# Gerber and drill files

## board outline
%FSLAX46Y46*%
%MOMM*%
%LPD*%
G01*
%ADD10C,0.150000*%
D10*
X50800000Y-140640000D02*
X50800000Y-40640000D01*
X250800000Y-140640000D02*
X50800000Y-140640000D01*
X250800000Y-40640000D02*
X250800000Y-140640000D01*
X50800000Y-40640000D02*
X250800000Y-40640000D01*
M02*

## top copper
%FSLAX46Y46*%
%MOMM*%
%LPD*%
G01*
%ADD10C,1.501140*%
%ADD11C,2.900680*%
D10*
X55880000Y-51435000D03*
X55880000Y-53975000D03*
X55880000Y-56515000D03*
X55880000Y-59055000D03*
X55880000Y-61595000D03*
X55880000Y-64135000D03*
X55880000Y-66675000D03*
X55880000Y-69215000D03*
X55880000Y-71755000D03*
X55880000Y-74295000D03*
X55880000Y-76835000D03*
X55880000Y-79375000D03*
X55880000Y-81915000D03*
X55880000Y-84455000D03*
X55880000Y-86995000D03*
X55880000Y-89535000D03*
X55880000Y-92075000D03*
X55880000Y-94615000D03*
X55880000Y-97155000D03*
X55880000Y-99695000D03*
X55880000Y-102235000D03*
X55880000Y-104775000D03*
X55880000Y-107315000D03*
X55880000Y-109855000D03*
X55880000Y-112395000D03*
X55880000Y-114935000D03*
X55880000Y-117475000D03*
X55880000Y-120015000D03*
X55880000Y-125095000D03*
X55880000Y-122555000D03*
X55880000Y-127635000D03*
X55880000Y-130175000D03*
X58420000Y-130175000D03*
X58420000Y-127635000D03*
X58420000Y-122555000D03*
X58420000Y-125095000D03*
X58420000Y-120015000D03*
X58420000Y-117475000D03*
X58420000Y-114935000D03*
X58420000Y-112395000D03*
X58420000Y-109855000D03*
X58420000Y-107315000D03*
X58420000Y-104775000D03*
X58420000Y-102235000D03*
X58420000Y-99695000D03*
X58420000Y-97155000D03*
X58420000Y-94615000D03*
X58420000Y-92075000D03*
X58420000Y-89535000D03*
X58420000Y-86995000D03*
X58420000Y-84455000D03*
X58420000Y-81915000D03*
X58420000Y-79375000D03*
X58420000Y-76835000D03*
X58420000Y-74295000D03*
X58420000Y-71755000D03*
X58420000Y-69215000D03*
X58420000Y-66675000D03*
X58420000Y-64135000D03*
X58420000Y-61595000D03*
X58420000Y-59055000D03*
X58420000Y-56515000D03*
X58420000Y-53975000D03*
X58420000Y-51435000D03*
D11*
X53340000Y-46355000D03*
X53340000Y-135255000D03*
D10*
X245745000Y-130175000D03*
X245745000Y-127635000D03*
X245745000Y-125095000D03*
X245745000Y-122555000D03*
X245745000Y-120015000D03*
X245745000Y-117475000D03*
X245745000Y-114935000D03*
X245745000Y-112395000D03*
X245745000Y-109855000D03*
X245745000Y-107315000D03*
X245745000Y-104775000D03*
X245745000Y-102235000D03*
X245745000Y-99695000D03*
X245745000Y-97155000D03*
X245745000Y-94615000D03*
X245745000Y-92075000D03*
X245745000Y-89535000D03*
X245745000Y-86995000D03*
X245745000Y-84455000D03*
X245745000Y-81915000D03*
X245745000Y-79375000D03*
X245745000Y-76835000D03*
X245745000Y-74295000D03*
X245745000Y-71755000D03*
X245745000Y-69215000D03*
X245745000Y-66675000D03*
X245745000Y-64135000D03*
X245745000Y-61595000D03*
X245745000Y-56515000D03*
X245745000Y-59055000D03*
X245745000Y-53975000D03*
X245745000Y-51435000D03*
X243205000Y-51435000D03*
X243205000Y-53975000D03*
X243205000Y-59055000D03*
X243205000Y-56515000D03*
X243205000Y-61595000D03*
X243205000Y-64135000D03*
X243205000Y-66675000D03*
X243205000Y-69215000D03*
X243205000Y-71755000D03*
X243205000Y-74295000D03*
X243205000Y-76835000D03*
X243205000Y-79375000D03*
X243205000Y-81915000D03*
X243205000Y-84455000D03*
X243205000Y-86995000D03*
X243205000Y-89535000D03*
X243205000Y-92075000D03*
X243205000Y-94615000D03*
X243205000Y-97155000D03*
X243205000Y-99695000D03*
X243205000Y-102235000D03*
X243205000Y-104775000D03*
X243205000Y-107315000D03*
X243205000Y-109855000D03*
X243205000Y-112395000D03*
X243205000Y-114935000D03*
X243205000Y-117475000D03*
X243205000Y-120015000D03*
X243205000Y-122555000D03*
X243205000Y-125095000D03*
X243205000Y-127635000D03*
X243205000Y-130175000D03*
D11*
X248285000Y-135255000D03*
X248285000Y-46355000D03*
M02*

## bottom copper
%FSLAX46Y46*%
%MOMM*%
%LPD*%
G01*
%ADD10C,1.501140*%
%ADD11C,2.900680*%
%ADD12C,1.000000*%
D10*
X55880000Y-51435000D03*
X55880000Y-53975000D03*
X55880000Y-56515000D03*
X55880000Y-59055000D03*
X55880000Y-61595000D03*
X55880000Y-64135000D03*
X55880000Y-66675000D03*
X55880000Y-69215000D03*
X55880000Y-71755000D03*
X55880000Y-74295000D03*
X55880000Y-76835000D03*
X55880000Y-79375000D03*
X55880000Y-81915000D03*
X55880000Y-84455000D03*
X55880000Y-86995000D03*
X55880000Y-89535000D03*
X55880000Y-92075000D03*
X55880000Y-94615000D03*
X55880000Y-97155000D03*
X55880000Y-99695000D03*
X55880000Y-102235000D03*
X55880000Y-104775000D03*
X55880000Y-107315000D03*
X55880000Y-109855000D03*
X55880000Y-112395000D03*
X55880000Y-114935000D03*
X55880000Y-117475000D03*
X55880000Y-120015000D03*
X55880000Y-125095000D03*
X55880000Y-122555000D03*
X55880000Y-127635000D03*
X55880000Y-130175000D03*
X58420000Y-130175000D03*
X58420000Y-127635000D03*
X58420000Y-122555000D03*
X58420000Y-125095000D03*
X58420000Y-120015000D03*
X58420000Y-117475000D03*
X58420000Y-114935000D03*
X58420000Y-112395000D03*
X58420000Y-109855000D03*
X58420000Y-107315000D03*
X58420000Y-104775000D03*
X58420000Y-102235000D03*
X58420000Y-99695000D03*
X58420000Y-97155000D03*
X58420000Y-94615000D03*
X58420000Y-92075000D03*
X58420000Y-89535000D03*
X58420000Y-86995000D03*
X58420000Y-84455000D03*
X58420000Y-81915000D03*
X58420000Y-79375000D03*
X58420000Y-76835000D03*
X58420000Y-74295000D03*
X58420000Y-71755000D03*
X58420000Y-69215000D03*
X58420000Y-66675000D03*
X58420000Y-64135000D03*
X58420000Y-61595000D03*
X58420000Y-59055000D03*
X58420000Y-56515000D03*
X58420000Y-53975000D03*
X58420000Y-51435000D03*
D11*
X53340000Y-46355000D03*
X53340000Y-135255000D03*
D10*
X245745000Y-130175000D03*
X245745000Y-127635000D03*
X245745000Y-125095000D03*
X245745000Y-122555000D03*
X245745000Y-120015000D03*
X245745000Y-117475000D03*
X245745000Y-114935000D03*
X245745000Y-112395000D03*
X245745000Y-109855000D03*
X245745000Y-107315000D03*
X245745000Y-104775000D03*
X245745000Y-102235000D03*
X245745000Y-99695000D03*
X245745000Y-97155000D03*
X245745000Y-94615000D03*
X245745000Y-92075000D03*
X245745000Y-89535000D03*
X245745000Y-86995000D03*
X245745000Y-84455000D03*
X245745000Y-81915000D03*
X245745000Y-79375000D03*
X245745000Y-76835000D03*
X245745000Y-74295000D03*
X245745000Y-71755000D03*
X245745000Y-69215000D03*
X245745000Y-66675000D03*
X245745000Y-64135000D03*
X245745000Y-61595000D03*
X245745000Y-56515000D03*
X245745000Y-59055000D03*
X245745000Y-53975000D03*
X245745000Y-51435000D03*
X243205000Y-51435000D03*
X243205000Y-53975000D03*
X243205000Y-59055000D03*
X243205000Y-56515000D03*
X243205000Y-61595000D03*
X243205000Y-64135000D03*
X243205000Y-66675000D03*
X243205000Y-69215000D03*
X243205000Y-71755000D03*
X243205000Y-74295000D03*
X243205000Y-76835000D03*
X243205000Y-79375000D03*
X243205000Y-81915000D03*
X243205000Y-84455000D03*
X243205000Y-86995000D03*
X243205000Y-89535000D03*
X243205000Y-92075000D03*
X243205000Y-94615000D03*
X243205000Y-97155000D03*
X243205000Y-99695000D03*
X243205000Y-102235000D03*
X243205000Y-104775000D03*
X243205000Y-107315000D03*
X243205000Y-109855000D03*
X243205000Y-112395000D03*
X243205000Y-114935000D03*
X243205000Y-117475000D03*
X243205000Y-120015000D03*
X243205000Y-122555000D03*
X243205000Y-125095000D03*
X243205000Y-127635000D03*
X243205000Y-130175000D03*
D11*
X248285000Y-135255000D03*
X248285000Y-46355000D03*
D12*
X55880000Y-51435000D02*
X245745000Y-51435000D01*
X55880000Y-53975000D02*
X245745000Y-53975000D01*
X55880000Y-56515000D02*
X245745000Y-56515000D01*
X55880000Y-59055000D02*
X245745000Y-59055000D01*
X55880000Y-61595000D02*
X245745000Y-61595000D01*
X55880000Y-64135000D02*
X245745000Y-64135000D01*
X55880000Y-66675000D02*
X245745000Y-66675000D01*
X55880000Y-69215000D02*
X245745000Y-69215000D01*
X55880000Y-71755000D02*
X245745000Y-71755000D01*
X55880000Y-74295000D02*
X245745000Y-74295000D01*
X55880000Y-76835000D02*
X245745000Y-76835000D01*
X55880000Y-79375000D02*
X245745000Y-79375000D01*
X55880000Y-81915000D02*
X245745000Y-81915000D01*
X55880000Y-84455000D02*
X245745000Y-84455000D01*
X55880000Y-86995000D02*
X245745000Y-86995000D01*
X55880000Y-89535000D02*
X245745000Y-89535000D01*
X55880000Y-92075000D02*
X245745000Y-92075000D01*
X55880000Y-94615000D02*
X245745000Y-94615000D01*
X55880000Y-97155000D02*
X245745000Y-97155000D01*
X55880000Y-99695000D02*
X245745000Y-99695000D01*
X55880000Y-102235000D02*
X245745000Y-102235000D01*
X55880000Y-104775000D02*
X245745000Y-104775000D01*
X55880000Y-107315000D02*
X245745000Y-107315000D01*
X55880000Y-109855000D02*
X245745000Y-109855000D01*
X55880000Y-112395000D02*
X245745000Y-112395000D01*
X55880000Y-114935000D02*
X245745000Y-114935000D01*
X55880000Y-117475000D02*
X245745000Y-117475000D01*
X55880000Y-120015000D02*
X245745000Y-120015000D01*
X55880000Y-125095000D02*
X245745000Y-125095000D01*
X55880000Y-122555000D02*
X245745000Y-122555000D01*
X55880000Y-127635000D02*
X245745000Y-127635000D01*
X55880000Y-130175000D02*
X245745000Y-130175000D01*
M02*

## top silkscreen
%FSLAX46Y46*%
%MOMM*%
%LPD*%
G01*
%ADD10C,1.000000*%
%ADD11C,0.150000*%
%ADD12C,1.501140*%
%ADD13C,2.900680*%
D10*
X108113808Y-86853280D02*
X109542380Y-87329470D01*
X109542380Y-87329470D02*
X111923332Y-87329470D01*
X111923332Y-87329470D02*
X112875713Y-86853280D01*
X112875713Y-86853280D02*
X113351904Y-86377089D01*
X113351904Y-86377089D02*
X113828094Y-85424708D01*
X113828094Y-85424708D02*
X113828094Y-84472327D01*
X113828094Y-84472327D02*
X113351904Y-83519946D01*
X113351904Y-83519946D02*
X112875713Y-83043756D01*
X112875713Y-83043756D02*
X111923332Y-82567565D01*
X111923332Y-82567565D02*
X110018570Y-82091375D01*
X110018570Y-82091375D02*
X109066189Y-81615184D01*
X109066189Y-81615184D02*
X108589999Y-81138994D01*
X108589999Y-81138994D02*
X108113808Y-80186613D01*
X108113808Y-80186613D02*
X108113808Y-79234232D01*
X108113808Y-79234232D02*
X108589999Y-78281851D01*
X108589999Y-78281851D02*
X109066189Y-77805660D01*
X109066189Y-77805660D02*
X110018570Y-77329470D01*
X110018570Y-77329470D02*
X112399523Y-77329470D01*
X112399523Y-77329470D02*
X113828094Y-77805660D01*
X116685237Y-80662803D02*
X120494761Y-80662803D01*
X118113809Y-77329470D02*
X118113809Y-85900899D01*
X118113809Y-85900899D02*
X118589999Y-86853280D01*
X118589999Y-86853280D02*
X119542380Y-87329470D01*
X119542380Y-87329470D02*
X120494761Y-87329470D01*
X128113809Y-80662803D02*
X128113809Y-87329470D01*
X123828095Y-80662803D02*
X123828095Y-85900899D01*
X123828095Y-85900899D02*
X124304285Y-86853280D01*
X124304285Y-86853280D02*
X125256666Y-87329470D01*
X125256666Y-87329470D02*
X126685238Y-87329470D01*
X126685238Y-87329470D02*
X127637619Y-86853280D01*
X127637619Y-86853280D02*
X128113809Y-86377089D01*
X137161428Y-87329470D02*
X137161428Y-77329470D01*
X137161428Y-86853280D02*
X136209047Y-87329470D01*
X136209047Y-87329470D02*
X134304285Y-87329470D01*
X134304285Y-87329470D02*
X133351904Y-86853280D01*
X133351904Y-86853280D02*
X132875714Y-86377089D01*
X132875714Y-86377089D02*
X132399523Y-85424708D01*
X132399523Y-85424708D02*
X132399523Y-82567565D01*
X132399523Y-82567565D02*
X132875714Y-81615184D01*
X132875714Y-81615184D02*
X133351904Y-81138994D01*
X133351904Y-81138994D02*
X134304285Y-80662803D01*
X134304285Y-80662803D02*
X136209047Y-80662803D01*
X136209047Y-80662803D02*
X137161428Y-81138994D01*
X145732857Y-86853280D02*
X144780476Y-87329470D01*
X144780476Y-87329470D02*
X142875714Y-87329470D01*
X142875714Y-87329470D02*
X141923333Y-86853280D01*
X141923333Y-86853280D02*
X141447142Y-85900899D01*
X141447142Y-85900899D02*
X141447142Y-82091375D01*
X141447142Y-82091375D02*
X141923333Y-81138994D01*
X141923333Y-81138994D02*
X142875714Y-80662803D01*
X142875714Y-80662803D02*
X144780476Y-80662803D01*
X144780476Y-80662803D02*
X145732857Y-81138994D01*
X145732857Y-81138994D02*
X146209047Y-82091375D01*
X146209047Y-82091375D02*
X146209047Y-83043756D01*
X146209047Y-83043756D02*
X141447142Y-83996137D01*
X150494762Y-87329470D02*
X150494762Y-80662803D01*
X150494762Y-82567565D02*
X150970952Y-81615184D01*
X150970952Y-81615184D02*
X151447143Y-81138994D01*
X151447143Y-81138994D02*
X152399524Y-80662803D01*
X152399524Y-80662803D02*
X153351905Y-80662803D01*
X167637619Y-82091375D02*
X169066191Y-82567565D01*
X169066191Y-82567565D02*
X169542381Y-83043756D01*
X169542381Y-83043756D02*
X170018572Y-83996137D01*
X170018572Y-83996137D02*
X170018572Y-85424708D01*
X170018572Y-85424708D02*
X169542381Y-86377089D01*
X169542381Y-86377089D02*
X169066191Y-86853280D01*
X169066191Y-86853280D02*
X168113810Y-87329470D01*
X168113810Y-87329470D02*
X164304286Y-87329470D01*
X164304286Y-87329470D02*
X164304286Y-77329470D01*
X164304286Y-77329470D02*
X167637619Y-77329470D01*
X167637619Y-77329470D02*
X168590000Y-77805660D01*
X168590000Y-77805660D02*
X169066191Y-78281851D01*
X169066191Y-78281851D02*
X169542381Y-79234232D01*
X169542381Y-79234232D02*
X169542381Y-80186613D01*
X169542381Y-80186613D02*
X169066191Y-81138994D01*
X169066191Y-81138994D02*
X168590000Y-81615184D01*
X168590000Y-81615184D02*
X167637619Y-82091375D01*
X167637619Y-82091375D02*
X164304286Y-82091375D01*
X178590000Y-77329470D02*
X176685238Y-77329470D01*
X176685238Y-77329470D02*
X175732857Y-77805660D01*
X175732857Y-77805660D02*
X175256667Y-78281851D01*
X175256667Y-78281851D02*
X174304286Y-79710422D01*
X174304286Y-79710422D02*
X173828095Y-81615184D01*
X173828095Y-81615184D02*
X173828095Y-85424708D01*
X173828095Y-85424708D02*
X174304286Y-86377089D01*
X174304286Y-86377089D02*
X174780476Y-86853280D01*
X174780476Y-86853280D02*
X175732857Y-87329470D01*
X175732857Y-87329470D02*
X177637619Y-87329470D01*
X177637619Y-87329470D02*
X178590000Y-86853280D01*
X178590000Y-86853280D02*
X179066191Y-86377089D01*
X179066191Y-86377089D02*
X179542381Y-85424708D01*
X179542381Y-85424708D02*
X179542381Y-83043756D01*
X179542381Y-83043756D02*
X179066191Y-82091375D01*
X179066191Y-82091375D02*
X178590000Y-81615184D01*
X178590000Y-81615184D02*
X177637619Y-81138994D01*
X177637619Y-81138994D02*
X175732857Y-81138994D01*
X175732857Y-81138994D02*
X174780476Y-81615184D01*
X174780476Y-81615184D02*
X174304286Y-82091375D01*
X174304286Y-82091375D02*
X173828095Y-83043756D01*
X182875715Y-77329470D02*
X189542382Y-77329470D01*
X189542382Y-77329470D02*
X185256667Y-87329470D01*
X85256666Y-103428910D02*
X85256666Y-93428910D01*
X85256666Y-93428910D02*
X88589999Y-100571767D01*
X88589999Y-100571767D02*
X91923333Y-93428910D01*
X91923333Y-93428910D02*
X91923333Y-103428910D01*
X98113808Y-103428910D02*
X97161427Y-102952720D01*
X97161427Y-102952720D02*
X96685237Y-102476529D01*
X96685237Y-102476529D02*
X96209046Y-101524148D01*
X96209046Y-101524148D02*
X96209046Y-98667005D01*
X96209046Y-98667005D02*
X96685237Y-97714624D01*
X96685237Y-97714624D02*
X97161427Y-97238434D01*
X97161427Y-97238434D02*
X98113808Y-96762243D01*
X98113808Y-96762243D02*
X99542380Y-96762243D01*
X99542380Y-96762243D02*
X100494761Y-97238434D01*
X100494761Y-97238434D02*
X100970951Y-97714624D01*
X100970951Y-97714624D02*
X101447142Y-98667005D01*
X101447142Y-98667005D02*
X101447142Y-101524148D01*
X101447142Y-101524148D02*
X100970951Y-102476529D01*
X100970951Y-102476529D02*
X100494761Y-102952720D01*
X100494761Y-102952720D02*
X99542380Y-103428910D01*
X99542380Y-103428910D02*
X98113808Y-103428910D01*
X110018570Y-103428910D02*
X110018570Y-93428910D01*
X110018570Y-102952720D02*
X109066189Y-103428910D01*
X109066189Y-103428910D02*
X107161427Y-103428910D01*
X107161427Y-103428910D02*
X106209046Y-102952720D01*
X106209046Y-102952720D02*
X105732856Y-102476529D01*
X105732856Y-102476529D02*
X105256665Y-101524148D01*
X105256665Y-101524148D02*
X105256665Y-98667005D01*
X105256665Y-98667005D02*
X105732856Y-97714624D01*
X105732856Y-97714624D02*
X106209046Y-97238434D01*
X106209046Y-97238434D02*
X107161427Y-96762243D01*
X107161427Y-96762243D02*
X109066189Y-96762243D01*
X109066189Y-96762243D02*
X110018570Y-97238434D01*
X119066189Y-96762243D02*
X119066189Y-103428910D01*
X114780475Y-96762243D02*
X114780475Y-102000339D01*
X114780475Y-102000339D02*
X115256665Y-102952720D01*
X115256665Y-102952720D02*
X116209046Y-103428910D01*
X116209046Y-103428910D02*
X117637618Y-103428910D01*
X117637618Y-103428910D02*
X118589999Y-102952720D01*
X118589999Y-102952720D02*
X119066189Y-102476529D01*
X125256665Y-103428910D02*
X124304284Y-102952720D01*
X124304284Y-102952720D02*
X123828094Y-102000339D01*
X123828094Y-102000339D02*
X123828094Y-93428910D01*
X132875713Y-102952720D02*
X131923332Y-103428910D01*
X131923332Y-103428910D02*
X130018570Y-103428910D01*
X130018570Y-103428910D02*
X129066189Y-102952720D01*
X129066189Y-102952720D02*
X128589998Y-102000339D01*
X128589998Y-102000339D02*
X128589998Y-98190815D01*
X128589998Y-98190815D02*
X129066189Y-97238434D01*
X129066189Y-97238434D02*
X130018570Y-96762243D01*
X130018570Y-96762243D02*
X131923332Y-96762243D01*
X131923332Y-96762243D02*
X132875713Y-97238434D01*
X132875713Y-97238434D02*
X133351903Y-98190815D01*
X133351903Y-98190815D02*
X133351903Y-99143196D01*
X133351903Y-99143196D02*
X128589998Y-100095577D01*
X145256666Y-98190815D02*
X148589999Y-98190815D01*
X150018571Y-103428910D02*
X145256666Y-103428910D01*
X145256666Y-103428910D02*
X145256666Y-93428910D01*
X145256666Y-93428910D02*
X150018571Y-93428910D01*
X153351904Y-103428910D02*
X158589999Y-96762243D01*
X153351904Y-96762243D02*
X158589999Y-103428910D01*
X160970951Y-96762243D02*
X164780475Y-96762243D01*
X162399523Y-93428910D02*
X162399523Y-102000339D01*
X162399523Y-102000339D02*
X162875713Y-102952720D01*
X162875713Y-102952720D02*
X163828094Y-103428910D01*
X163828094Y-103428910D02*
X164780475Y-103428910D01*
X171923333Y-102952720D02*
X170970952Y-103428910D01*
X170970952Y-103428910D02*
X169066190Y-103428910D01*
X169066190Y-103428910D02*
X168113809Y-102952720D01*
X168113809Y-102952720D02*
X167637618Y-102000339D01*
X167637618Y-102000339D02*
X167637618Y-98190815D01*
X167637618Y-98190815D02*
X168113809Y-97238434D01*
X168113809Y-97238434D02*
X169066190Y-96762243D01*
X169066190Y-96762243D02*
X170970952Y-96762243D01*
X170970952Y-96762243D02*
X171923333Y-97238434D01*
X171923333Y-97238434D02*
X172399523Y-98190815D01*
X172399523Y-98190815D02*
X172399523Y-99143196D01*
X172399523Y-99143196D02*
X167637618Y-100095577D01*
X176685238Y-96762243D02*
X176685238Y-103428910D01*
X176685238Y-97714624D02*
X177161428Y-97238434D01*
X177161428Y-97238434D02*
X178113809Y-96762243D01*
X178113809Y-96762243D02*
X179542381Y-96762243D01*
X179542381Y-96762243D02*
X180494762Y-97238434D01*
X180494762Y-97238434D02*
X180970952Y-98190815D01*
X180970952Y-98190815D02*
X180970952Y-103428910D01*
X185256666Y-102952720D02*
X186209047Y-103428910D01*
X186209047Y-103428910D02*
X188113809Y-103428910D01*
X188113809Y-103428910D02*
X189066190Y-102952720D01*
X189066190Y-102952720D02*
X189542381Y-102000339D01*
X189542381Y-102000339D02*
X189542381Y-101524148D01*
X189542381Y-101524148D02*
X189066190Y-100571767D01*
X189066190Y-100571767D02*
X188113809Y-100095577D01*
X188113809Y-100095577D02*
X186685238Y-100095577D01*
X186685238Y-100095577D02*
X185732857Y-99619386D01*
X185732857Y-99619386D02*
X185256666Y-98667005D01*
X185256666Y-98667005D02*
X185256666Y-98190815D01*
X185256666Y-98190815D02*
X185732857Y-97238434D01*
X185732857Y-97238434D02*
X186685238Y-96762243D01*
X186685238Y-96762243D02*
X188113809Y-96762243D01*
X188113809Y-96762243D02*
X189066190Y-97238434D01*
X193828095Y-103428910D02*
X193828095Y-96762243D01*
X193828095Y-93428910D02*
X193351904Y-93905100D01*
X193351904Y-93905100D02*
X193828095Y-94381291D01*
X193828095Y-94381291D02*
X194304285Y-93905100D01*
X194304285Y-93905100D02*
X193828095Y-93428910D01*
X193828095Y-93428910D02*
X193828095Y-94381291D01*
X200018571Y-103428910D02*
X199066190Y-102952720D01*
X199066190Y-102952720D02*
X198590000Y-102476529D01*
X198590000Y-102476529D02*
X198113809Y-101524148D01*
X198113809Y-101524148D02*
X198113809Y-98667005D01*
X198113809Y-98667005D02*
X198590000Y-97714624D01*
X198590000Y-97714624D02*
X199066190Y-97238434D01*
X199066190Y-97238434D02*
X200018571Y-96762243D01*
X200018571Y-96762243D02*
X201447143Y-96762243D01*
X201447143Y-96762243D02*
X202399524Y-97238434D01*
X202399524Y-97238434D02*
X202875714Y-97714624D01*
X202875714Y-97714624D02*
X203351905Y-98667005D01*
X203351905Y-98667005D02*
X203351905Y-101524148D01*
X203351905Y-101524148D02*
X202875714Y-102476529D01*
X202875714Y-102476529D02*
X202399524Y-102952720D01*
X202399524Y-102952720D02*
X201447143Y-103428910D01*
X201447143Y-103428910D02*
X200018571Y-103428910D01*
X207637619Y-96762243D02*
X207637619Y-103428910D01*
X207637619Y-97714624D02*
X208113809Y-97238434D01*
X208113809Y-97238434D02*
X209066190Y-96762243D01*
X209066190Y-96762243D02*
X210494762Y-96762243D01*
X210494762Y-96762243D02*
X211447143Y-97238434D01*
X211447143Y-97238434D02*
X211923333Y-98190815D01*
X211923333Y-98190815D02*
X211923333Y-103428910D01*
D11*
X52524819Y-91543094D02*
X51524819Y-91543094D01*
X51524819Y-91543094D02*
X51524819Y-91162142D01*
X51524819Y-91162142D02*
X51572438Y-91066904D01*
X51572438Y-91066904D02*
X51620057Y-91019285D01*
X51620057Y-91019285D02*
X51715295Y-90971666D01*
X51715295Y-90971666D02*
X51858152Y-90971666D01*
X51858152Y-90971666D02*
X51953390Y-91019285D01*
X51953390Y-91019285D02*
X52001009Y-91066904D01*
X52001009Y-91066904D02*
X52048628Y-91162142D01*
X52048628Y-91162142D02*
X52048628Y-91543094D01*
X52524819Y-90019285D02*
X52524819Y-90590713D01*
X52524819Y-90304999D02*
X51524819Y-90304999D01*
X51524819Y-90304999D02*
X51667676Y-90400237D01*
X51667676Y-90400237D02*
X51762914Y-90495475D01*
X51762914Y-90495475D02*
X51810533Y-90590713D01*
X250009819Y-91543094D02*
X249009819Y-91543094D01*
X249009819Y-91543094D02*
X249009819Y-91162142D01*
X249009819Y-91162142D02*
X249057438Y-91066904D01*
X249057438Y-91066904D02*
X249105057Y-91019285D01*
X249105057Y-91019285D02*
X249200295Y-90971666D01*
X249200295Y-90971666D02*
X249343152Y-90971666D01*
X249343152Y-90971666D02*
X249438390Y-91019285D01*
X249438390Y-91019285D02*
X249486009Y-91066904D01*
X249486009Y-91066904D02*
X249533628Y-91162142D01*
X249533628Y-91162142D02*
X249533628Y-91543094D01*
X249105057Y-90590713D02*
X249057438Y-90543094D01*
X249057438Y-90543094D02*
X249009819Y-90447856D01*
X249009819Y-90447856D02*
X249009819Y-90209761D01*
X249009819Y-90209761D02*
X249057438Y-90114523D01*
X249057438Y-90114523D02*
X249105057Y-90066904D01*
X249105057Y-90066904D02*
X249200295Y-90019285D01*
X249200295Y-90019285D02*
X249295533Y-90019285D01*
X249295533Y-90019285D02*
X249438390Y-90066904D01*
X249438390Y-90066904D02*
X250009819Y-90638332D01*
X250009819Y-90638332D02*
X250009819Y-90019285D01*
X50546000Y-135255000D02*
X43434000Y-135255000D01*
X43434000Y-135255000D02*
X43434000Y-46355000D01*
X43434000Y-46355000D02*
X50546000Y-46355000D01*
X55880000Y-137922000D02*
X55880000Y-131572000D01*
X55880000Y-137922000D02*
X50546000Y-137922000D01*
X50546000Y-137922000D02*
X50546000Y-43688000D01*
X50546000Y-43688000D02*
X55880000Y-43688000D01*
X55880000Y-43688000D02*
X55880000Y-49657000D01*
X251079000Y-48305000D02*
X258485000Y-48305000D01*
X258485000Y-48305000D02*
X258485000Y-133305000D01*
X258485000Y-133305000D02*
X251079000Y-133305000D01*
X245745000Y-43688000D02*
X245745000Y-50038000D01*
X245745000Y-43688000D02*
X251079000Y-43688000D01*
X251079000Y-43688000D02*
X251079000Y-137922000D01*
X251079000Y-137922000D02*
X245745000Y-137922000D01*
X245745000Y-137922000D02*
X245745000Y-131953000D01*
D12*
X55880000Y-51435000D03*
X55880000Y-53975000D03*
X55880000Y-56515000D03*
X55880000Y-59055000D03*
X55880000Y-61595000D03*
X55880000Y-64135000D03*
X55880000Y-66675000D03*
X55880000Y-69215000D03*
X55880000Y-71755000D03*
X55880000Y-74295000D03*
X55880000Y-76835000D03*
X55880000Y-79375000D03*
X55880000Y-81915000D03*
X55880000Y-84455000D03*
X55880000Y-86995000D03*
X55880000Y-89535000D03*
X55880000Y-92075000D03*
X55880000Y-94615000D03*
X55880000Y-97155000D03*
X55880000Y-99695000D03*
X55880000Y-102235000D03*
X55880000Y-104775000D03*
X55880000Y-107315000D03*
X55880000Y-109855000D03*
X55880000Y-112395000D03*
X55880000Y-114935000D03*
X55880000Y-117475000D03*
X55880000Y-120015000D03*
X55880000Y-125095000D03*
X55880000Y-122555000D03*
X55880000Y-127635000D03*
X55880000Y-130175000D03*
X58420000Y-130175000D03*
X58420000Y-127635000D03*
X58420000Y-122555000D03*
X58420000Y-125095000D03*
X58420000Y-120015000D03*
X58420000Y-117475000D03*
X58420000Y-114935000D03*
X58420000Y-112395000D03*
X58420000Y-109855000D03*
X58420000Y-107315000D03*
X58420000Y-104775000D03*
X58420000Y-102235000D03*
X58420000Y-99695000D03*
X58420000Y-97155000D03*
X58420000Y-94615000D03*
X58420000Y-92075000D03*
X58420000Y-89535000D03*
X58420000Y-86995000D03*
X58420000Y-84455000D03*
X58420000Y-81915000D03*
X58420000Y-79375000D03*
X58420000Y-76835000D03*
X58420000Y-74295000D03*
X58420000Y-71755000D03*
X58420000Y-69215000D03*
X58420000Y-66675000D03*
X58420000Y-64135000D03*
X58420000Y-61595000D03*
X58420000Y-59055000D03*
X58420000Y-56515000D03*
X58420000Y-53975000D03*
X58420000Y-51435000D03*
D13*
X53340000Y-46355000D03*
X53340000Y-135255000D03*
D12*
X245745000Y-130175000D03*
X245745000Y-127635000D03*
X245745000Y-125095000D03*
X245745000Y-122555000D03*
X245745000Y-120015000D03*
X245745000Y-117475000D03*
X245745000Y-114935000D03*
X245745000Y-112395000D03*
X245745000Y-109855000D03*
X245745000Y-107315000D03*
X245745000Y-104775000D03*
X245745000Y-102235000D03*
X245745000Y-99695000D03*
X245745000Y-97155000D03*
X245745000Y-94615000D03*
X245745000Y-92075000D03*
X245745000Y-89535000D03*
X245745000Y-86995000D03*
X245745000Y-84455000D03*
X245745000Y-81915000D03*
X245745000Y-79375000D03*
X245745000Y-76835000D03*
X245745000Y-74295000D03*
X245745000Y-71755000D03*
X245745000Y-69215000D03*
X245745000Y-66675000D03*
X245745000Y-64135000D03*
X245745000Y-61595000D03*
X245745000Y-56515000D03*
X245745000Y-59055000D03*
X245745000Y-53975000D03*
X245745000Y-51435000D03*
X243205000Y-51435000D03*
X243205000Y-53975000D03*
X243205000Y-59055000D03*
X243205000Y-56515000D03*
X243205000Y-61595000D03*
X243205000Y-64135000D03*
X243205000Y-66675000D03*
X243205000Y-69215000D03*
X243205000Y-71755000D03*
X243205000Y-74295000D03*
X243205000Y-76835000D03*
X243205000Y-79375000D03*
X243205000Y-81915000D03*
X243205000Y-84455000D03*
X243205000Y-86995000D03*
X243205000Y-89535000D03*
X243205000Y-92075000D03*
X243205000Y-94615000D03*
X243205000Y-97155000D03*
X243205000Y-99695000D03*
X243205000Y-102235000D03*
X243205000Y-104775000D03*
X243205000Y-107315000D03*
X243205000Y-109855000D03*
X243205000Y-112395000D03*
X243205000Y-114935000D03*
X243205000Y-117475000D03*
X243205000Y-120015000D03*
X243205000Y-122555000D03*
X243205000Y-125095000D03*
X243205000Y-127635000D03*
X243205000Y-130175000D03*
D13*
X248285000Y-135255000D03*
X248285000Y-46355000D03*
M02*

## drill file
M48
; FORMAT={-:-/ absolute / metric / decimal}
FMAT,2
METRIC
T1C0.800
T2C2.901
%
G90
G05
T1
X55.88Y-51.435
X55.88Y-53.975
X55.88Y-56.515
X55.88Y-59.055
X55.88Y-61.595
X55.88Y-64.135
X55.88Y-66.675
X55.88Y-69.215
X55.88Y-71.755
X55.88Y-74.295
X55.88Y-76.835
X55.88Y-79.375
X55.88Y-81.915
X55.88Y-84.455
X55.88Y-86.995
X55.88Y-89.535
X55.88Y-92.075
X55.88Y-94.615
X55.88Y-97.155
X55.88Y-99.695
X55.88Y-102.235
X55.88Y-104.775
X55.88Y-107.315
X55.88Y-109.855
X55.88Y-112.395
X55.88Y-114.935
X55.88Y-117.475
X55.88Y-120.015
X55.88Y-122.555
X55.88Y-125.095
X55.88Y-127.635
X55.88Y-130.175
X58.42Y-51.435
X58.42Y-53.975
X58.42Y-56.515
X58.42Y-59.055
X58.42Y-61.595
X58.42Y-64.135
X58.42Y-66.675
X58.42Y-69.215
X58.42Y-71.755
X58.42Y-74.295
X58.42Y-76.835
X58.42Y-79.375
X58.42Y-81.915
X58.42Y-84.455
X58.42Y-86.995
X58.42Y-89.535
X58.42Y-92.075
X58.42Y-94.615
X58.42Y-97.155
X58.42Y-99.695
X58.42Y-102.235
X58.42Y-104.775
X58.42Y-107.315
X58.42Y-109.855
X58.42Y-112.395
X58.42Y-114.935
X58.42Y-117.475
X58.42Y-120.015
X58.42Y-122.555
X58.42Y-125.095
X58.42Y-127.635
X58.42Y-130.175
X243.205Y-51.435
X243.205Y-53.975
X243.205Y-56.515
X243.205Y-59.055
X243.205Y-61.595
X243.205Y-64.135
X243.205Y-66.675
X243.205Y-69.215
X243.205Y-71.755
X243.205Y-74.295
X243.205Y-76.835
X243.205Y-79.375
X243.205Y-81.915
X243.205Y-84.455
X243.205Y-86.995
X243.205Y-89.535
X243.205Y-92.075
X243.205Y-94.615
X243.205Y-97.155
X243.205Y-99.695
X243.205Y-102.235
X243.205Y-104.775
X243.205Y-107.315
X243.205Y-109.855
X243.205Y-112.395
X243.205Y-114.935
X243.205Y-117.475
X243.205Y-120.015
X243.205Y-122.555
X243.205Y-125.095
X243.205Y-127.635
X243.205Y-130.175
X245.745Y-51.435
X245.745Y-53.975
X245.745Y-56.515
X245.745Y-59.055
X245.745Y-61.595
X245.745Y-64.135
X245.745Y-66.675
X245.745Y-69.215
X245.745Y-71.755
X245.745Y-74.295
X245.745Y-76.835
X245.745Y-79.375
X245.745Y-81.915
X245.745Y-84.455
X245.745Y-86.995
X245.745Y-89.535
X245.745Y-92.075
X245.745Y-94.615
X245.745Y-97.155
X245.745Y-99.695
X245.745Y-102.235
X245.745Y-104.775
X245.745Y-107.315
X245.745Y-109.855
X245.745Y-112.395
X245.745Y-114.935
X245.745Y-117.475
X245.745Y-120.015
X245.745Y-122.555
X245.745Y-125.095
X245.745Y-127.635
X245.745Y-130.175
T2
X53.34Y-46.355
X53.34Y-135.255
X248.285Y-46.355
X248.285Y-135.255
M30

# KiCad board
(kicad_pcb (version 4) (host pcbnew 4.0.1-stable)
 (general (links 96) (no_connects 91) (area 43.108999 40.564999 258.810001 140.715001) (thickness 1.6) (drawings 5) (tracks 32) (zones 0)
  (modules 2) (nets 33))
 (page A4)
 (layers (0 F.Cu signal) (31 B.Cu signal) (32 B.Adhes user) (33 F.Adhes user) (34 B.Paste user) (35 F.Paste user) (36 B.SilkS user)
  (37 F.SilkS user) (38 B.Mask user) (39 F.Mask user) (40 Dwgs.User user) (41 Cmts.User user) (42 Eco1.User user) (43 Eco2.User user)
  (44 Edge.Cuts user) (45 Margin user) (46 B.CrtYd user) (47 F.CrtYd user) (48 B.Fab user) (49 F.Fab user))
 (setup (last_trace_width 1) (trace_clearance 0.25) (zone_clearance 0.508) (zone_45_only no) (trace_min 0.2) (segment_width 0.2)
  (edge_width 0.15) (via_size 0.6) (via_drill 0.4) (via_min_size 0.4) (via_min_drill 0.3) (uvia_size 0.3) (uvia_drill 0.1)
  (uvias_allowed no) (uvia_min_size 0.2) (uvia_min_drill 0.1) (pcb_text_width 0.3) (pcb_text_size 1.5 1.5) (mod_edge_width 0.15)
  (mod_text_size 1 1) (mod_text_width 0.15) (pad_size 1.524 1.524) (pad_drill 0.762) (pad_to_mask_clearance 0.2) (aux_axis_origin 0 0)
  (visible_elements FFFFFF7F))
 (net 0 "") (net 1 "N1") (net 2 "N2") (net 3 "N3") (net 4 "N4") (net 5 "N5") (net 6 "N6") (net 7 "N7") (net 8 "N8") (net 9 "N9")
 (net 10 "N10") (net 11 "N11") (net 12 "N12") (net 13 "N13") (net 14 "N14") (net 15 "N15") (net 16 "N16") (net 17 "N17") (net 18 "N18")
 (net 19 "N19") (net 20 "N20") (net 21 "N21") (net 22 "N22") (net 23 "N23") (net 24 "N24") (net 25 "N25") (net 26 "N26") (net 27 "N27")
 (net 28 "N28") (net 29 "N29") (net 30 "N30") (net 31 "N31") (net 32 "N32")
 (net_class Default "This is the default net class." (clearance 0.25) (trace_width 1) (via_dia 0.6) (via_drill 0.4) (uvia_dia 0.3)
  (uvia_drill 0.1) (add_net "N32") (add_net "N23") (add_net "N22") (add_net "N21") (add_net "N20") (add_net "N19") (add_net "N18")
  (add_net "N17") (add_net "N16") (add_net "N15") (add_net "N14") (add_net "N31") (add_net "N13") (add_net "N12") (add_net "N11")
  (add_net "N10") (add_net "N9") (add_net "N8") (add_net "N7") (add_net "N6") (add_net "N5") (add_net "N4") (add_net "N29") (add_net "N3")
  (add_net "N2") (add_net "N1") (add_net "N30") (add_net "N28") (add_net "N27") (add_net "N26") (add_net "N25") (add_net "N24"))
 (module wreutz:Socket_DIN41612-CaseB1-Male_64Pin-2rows (layer F.Cu) (at 57.15 90.805 270)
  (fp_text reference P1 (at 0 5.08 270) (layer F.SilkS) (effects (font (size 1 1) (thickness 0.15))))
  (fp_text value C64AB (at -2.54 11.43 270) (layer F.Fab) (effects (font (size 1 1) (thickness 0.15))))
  (fp_line (start 44.45 6.604) (end 44.45 13.716) (layer F.SilkS) (width 0.15))
  (fp_line (start 44.45 13.716) (end -44.45 13.716) (layer F.SilkS) (width 0.15))
  (fp_line (start -44.45 13.716) (end -44.45 6.604) (layer F.SilkS) (width 0.15))
  (fp_line (start 47.117 1.27) (end 40.767 1.27) (layer F.SilkS) (width 0.15))
  (fp_line (start 47.117 1.27) (end 47.117 6.604) (layer F.SilkS) (width 0.15))
  (fp_line (start 47.117 6.604) (end -47.117 6.604) (layer F.SilkS) (width 0.15))
  (fp_line (start -47.117 6.604) (end -47.117 1.27) (layer F.SilkS) (width 0.15))
  (fp_line (start -47.117 1.27) (end -41.148 1.27) (layer F.SilkS) (width 0.15))
  (pad B32 thru_hole circle (at -39.37 1.27 90) (size 1.50114 1.50114) (drill 0.8001) (layers *.Cu *.Mask F.SilkS) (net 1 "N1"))
  (pad B31 thru_hole circle (at -36.83 1.27 90) (size 1.50114 1.50114) (drill 0.8001) (layers *.Cu *.Mask F.SilkS) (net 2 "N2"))
  (pad B30 thru_hole circle (at -34.29 1.27 90) (size 1.50114 1.50114) (drill 0.8001) (layers *.Cu *.Mask F.SilkS) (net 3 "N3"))
  (pad B29 thru_hole circle (at -31.75 1.27 90) (size 1.50114 1.50114) (drill 0.8001) (layers *.Cu *.Mask F.SilkS) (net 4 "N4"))
  (pad B28 thru_hole circle (at -29.21 1.27 90) (size 1.50114 1.50114) (drill 0.8001) (layers *.Cu *.Mask F.SilkS) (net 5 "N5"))
  (pad B27 thru_hole circle (at -26.67 1.27 90) (size 1.50114 1.50114) (drill 0.8001) (layers *.Cu *.Mask F.SilkS) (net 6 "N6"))
  (pad B26 thru_hole circle (at -24.13 1.27 90) (size 1.50114 1.50114) (drill 0.8001) (layers *.Cu *.Mask F.SilkS) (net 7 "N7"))
  (pad B25 thru_hole circle (at -21.59 1.27 90) (size 1.50114 1.50114) (drill 0.8001) (layers *.Cu *.Mask F.SilkS) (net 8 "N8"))
  (pad B24 thru_hole circle (at -19.05 1.27 90) (size 1.50114 1.50114) (drill 0.8001) (layers *.Cu *.Mask F.SilkS) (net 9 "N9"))
  (pad B23 thru_hole circle (at -16.51 1.27 90) (size 1.50114 1.50114) (drill 0.8001) (layers *.Cu *.Mask F.SilkS) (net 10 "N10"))
  (pad B22 thru_hole circle (at -13.97 1.27 90) (size 1.50114 1.50114) (drill 0.8001) (layers *.Cu *.Mask F.SilkS) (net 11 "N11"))
  (pad B21 thru_hole circle (at -11.43 1.27 90) (size 1.50114 1.50114) (drill 0.8001) (layers *.Cu *.Mask F.SilkS) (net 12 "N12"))
  (pad B20 thru_hole circle (at -8.89 1.27 90) (size 1.50114 1.50114) (drill 0.8001) (layers *.Cu *.Mask F.SilkS) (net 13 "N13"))
  (pad B19 thru_hole circle (at -6.35 1.27 90) (size 1.50114 1.50114) (drill 0.8001) (layers *.Cu *.Mask F.SilkS) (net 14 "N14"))
  (pad B18 thru_hole circle (at -3.81 1.27 90) (size 1.50114 1.50114) (drill 0.8001) (layers *.Cu *.Mask F.SilkS) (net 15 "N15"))
  (pad B17 thru_hole circle (at -1.27 1.27 90) (size 1.50114 1.50114) (drill 0.8001) (layers *.Cu *.Mask F.SilkS) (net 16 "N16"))
  (pad B16 thru_hole circle (at 1.27 1.27 90) (size 1.50114 1.50114) (drill 0.8001) (layers *.Cu *.Mask F.SilkS) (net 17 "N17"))
  (pad B15 thru_hole circle (at 3.81 1.27 90) (size 1.50114 1.50114) (drill 0.8001) (layers *.Cu *.Mask F.SilkS) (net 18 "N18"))
  (pad B14 thru_hole circle (at 6.35 1.27 90) (size 1.50114 1.50114) (drill 0.8001) (layers *.Cu *.Mask F.SilkS) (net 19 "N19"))
  (pad B13 thru_hole circle (at 8.89 1.27 90) (size 1.50114 1.50114) (drill 0.8001) (layers *.Cu *.Mask F.SilkS) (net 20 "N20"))
  (pad B12 thru_hole circle (at 11.43 1.27 90) (size 1.50114 1.50114) (drill 0.8001) (layers *.Cu *.Mask F.SilkS) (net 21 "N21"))
  (pad B11 thru_hole circle (at 13.97 1.27 90) (size 1.50114 1.50114) (drill 0.8001) (layers *.Cu *.Mask F.SilkS) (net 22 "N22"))
  (pad B10 thru_hole circle (at 16.51 1.27 90) (size 1.50114 1.50114) (drill 0.8001) (layers *.Cu *.Mask F.SilkS) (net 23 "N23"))
  (pad B9 thru_hole circle (at 19.05 1.27 90) (size 1.50114 1.50114) (drill 0.8001) (layers *.Cu *.Mask F.SilkS) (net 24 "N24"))
  (pad B8 thru_hole circle (at 21.59 1.27 90) (size 1.50114 1.50114) (drill 0.8001) (layers *.Cu *.Mask F.SilkS) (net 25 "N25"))
  (pad B7 thru_hole circle (at 24.13 1.27 90) (size 1.50114 1.50114) (drill 0.8001) (layers *.Cu *.Mask F.SilkS) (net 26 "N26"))
  (pad B6 thru_hole circle (at 26.67 1.27 90) (size 1.50114 1.50114) (drill 0.8001) (layers *.Cu *.Mask F.SilkS) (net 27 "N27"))
  (pad B5 thru_hole circle (at 29.21 1.27 90) (size 1.50114 1.50114) (drill 0.8001) (layers *.Cu *.Mask F.SilkS) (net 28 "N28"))
  (pad B3 thru_hole circle (at 34.29 1.27 90) (size 1.50114 1.50114) (drill 0.8001) (layers *.Cu *.Mask F.SilkS) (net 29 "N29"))
  (pad B4 thru_hole circle (at 31.75 1.27 90) (size 1.50114 1.50114) (drill 0.8001) (layers *.Cu *.Mask F.SilkS) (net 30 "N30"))
  (pad B2 thru_hole circle (at 36.83 1.27 90) (size 1.50114 1.50114) (drill 0.8001) (layers *.Cu *.Mask F.SilkS) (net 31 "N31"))
  (pad B1 thru_hole circle (at 39.37 1.27 90) (size 1.50114 1.50114) (drill 0.8001) (layers *.Cu *.Mask F.SilkS) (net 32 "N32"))
  (pad A1 thru_hole circle (at 39.37 -1.27 90) (size 1.50114 1.50114) (drill 0.8001) (layers *.Cu *.Mask F.SilkS) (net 32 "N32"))
  (pad A2 thru_hole circle (at 36.83 -1.27 90) (size 1.50114 1.50114) (drill 0.8001) (layers *.Cu *.Mask F.SilkS) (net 31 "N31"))
  (pad A4 thru_hole circle (at 31.75 -1.27 90) (size 1.50114 1.50114) (drill 0.8001) (layers *.Cu *.Mask F.SilkS) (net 30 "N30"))
  (pad A3 thru_hole circle (at 34.29 -1.27 90) (size 1.50114 1.50114) (drill 0.8001) (layers *.Cu *.Mask F.SilkS) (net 29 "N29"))
  (pad A5 thru_hole circle (at 29.21 -1.27 90) (size 1.50114 1.50114) (drill 0.8001) (layers *.Cu *.Mask F.SilkS) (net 28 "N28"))
  (pad A6 thru_hole circle (at 26.67 -1.27 90) (size 1.50114 1.50114) (drill 0.8001) (layers *.Cu *.Mask F.SilkS) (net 27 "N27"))
  (pad A7 thru_hole circle (at 24.13 -1.27 90) (size 1.50114 1.50114) (drill 0.8001) (layers *.Cu *.Mask F.SilkS) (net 26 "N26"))
  (pad A8 thru_hole circle (at 21.59 -1.27 90) (size 1.50114 1.50114) (drill 0.8001) (layers *.Cu *.Mask F.SilkS) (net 25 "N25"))
  (pad A9 thru_hole circle (at 19.05 -1.27 90) (size 1.50114 1.50114) (drill 0.8001) (layers *.Cu *.Mask F.SilkS) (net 24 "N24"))
  (pad A10 thru_hole circle (at 16.51 -1.27 90) (size 1.50114 1.50114) (drill 0.8001) (layers *.Cu *.Mask F.SilkS) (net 23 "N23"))
  (pad A11 thru_hole circle (at 13.97 -1.27 90) (size 1.50114 1.50114) (drill 0.8001) (layers *.Cu *.Mask F.SilkS) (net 22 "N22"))
  (pad A12 thru_hole circle (at 11.43 -1.27 90) (size 1.50114 1.50114) (drill 0.8001) (layers *.Cu *.Mask F.SilkS) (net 21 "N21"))
  (pad A13 thru_hole circle (at 8.89 -1.27 90) (size 1.50114 1.50114) (drill 0.8001) (layers *.Cu *.Mask F.SilkS) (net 20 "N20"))
  (pad A14 thru_hole circle (at 6.35 -1.27 90) (size 1.50114 1.50114) (drill 0.8001) (layers *.Cu *.Mask F.SilkS) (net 19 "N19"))
  (pad A15 thru_hole circle (at 3.81 -1.27 90) (size 1.50114 1.50114) (drill 0.8001) (layers *.Cu *.Mask F.SilkS) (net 18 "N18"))
  (pad A16 thru_hole circle (at 1.27 -1.27 90) (size 1.50114 1.50114) (drill 0.8001) (layers *.Cu *.Mask F.SilkS) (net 17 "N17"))
  (pad A17 thru_hole circle (at -1.27 -1.27 90) (size 1.50114 1.50114) (drill 0.8001) (layers *.Cu *.Mask F.SilkS) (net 16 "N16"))
  (pad A18 thru_hole circle (at -3.81 -1.27 90) (size 1.50114 1.50114) (drill 0.8001) (layers *.Cu *.Mask F.SilkS) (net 15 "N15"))
  (pad A19 thru_hole circle (at -6.35 -1.27 90) (size 1.50114 1.50114) (drill 0.8001) (layers *.Cu *.Mask F.SilkS) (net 14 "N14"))
  (pad A20 thru_hole circle (at -8.89 -1.27 90) (size 1.50114 1.50114) (drill 0.8001) (layers *.Cu *.Mask F.SilkS) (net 13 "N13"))
  (pad A21 thru_hole circle (at -11.43 -1.27 90) (size 1.50114 1.50114) (drill 0.8001) (layers *.Cu *.Mask F.SilkS) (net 12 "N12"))
  (pad A22 thru_hole circle (at -13.97 -1.27 90) (size 1.50114 1.50114) (drill 0.8001) (layers *.Cu *.Mask F.SilkS) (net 11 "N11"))
  (pad A23 thru_hole circle (at -16.51 -1.27 90) (size 1.50114 1.50114) (drill 0.8001) (layers *.Cu *.Mask F.SilkS) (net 10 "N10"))
  (pad A24 thru_hole circle (at -19.05 -1.27 90) (size 1.50114 1.50114) (drill 0.8001) (layers *.Cu *.Mask F.SilkS) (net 9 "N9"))
  (pad A25 thru_hole circle (at -21.59 -1.27 90) (size 1.50114 1.50114) (drill 0.8001) (layers *.Cu *.Mask F.SilkS) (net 8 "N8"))
  (pad A26 thru_hole circle (at -24.13 -1.27 90) (size 1.50114 1.50114) (drill 0.8001) (layers *.Cu *.Mask F.SilkS) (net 7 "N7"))
  (pad A27 thru_hole circle (at -26.67 -1.27 90) (size 1.50114 1.50114) (drill 0.8001) (layers *.Cu *.Mask F.SilkS) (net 6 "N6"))
  (pad A28 thru_hole circle (at -29.21 -1.27 90) (size 1.50114 1.50114) (drill 0.8001) (layers *.Cu *.Mask F.SilkS) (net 5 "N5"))
  (pad A29 thru_hole circle (at -31.75 -1.27 90) (size 1.50114 1.50114) (drill 0.8001) (layers *.Cu *.Mask F.SilkS) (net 4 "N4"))
  (pad A30 thru_hole circle (at -34.29 -1.27 90) (size 1.50114 1.50114) (drill 0.8001) (layers *.Cu *.Mask F.SilkS) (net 3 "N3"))
  (pad A31 thru_hole circle (at -36.83 -1.27 90) (size 1.50114 1.50114) (drill 0.8001) (layers *.Cu *.Mask F.SilkS) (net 2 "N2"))
  (pad A32 thru_hole circle (at -39.37 -1.27 90) (size 1.50114 1.50114) (drill 0.8001) (layers *.Cu *.Mask F.SilkS) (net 1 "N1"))
  (pad 1 thru_hole circle (at -44.45 3.81 270) (size 2.90068 2.90068) (drill 2.90068) (layers *.Cu *.Mask F.SilkS))
  (pad 1 thru_hole circle (at 44.45 3.81 270) (size 2.90068 2.90068) (drill 2.90068) (layers *.Cu *.Mask F.SilkS)))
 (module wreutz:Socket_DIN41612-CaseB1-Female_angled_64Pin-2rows (layer F.Cu) (at 244.475 90.805 90)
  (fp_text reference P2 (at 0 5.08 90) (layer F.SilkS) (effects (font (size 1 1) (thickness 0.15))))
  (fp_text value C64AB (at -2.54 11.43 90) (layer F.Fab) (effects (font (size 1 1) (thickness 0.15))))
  (fp_line (start 42.5 6.604) (end 42.5 14.01) (layer F.SilkS) (width 0.15))
  (fp_line (start 42.5 14.01) (end -42.5 14.01) (layer F.SilkS) (width 0.15))
  (fp_line (start -42.5 14.01) (end -42.5 6.604) (layer F.SilkS) (width 0.15))
  (fp_line (start 47.117 1.27) (end 40.767 1.27) (layer F.SilkS) (width 0.15))
  (fp_line (start 47.117 1.27) (end 47.117 6.604) (layer F.SilkS) (width 0.15))
  (fp_line (start 47.117 6.604) (end -47.117 6.604) (layer F.SilkS) (width 0.15))
  (fp_line (start -47.117 6.604) (end -47.117 1.27) (layer F.SilkS) (width 0.15))
  (fp_line (start -47.117 1.27) (end -41.148 1.27) (layer F.SilkS) (width 0.15))
  (pad B1 thru_hole circle (at -39.37 1.27 270) (size 1.50114 1.50114) (drill 0.8001) (layers *.Cu *.Mask F.SilkS) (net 32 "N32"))
  (pad B2 thru_hole circle (at -36.83 1.27 270) (size 1.50114 1.50114) (drill 0.8001) (layers *.Cu *.Mask F.SilkS) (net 31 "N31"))
  (pad B3 thru_hole circle (at -34.29 1.27 270) (size 1.50114 1.50114) (drill 0.8001) (layers *.Cu *.Mask F.SilkS) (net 29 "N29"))
  (pad B4 thru_hole circle (at -31.75 1.27 270) (size 1.50114 1.50114) (drill 0.8001) (layers *.Cu *.Mask F.SilkS) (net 30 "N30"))
  (pad B5 thru_hole circle (at -29.21 1.27 270) (size 1.50114 1.50114) (drill 0.8001) (layers *.Cu *.Mask F.SilkS) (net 28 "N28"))
  (pad B6 thru_hole circle (at -26.67 1.27 270) (size 1.50114 1.50114) (drill 0.8001) (layers *.Cu *.Mask F.SilkS) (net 27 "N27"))
  (pad B7 thru_hole circle (at -24.13 1.27 270) (size 1.50114 1.50114) (drill 0.8001) (layers *.Cu *.Mask F.SilkS) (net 26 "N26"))
  (pad B8 thru_hole circle (at -21.59 1.27 270) (size 1.50114 1.50114) (drill 0.8001) (layers *.Cu *.Mask F.SilkS) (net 25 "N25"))
  (pad B9 thru_hole circle (at -19.05 1.27 270) (size 1.50114 1.50114) (drill 0.8001) (layers *.Cu *.Mask F.SilkS) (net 24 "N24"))
  (pad B10 thru_hole circle (at -16.51 1.27 270) (size 1.50114 1.50114) (drill 0.8001) (layers *.Cu *.Mask F.SilkS) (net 23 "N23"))
  (pad B11 thru_hole circle (at -13.97 1.27 270) (size 1.50114 1.50114) (drill 0.8001) (layers *.Cu *.Mask F.SilkS) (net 22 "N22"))
  (pad B12 thru_hole circle (at -11.43 1.27 270) (size 1.50114 1.50114) (drill 0.8001) (layers *.Cu *.Mask F.SilkS) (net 21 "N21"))
  (pad B13 thru_hole circle (at -8.89 1.27 270) (size 1.50114 1.50114) (drill 0.8001) (layers *.Cu *.Mask F.SilkS) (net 20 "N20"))
  (pad B14 thru_hole circle (at -6.35 1.27 270) (size 1.50114 1.50114) (drill 0.8001) (layers *.Cu *.Mask F.SilkS) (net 19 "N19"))
  (pad B15 thru_hole circle (at -3.81 1.27 270) (size 1.50114 1.50114) (drill 0.8001) (layers *.Cu *.Mask F.SilkS) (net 18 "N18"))
  (pad B16 thru_hole circle (at -1.27 1.27 270) (size 1.50114 1.50114) (drill 0.8001) (layers *.Cu *.Mask F.SilkS) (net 17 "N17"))
  (pad B17 thru_hole circle (at 1.27 1.27 270) (size 1.50114 1.50114) (drill 0.8001) (layers *.Cu *.Mask F.SilkS) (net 16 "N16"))
  (pad B18 thru_hole circle (at 3.81 1.27 270) (size 1.50114 1.50114) (drill 0.8001) (layers *.Cu *.Mask F.SilkS) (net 15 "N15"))
  (pad B19 thru_hole circle (at 6.35 1.27 270) (size 1.50114 1.50114) (drill 0.8001) (layers *.Cu *.Mask F.SilkS) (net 14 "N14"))
  (pad B20 thru_hole circle (at 8.89 1.27 270) (size 1.50114 1.50114) (drill 0.8001) (layers *.Cu *.Mask F.SilkS) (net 13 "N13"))
  (pad B21 thru_hole circle (at 11.43 1.27 270) (size 1.50114 1.50114) (drill 0.8001) (layers *.Cu *.Mask F.SilkS) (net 12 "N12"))
  (pad B22 thru_hole circle (at 13.97 1.27 270) (size 1.50114 1.50114) (drill 0.8001) (layers *.Cu *.Mask F.SilkS) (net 11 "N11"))
  (pad B23 thru_hole circle (at 16.51 1.27 270) (size 1.50114 1.50114) (drill 0.8001) (layers *.Cu *.Mask F.SilkS) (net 10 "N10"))
  (pad B24 thru_hole circle (at 19.05 1.27 270) (size 1.50114 1.50114) (drill 0.8001) (layers *.Cu *.Mask F.SilkS) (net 9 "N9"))
  (pad B25 thru_hole circle (at 21.59 1.27 270) (size 1.50114 1.50114) (drill 0.8001) (layers *.Cu *.Mask F.SilkS) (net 8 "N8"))
  (pad B26 thru_hole circle (at 24.13 1.27 270) (size 1.50114 1.50114) (drill 0.8001) (layers *.Cu *.Mask F.SilkS) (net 7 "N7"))
  (pad B27 thru_hole circle (at 26.67 1.27 270) (size 1.50114 1.50114) (drill 0.8001) (layers *.Cu *.Mask F.SilkS) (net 6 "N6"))
  (pad B28 thru_hole circle (at 29.21 1.27 270) (size 1.50114 1.50114) (drill 0.8001) (layers *.Cu *.Mask F.SilkS) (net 5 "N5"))
  (pad B30 thru_hole circle (at 34.29 1.27 270) (size 1.50114 1.50114) (drill 0.8001) (layers *.Cu *.Mask F.SilkS) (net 3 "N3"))
  (pad B29 thru_hole circle (at 31.75 1.27 270) (size 1.50114 1.50114) (drill 0.8001) (layers *.Cu *.Mask F.SilkS) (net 4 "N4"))
  (pad B31 thru_hole circle (at 36.83 1.27 270) (size 1.50114 1.50114) (drill 0.8001) (layers *.Cu *.Mask F.SilkS) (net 2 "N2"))
  (pad B32 thru_hole circle (at 39.37 1.27 270) (size 1.50114 1.50114) (drill 0.8001) (layers *.Cu *.Mask F.SilkS) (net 1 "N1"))
  (pad A32 thru_hole circle (at 39.37 -1.27 270) (size 1.50114 1.50114) (drill 0.8001) (layers *.Cu *.Mask F.SilkS) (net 1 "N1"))
  (pad A31 thru_hole circle (at 36.83 -1.27 270) (size 1.50114 1.50114) (drill 0.8001) (layers *.Cu *.Mask F.SilkS) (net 2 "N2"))
  (pad A29 thru_hole circle (at 31.75 -1.27 270) (size 1.50114 1.50114) (drill 0.8001) (layers *.Cu *.Mask F.SilkS) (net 4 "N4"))
  (pad A30 thru_hole circle (at 34.29 -1.27 270) (size 1.50114 1.50114) (drill 0.8001) (layers *.Cu *.Mask F.SilkS) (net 3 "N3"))
  (pad A28 thru_hole circle (at 29.21 -1.27 270) (size 1.50114 1.50114) (drill 0.8001) (layers *.Cu *.Mask F.SilkS) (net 5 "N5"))
  (pad A27 thru_hole circle (at 26.67 -1.27 270) (size 1.50114 1.50114) (drill 0.8001) (layers *.Cu *.Mask F.SilkS) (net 6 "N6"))
  (pad A26 thru_hole circle (at 24.13 -1.27 270) (size 1.50114 1.50114) (drill 0.8001) (layers *.Cu *.Mask F.SilkS) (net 7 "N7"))
  (pad A25 thru_hole circle (at 21.59 -1.27 270) (size 1.50114 1.50114) (drill 0.8001) (layers *.Cu *.Mask F.SilkS) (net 8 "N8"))
  (pad A24 thru_hole circle (at 19.05 -1.27 270) (size 1.50114 1.50114) (drill 0.8001) (layers *.Cu *.Mask F.SilkS) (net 9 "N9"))
  (pad A23 thru_hole circle (at 16.51 -1.27 270) (size 1.50114 1.50114) (drill 0.8001) (layers *.Cu *.Mask F.SilkS) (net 10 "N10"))
  (pad A22 thru_hole circle (at 13.97 -1.27 270) (size 1.50114 1.50114) (drill 0.8001) (layers *.Cu *.Mask F.SilkS) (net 11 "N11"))
  (pad A21 thru_hole circle (at 11.43 -1.27 270) (size 1.50114 1.50114) (drill 0.8001) (layers *.Cu *.Mask F.SilkS) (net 12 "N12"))
  (pad A20 thru_hole circle (at 8.89 -1.27 270) (size 1.50114 1.50114) (drill 0.8001) (layers *.Cu *.Mask F.SilkS) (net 13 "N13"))
  (pad A19 thru_hole circle (at 6.35 -1.27 270) (size 1.50114 1.50114) (drill 0.8001) (layers *.Cu *.Mask F.SilkS) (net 14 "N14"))
  (pad A18 thru_hole circle (at 3.81 -1.27 270) (size 1.50114 1.50114) (drill 0.8001) (layers *.Cu *.Mask F.SilkS) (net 15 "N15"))
  (pad A17 thru_hole circle (at 1.27 -1.27 270) (size 1.50114 1.50114) (drill 0.8001) (layers *.Cu *.Mask F.SilkS) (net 16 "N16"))
  (pad A16 thru_hole circle (at -1.27 -1.27 270) (size 1.50114 1.50114) (drill 0.8001) (layers *.Cu *.Mask F.SilkS) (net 17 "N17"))
  (pad A15 thru_hole circle (at -3.81 -1.27 270) (size 1.50114 1.50114) (drill 0.8001) (layers *.Cu *.Mask F.SilkS) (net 18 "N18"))
  (pad A14 thru_hole circle (at -6.35 -1.27 270) (size 1.50114 1.50114) (drill 0.8001) (layers *.Cu *.Mask F.SilkS) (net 19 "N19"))
  (pad A13 thru_hole circle (at -8.89 -1.27 270) (size 1.50114 1.50114) (drill 0.8001) (layers *.Cu *.Mask F.SilkS) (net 20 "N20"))
  (pad A12 thru_hole circle (at -11.43 -1.27 270) (size 1.50114 1.50114) (drill 0.8001) (layers *.Cu *.Mask F.SilkS) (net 21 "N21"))
  (pad A11 thru_hole circle (at -13.97 -1.27 270) (size 1.50114 1.50114) (drill 0.8001) (layers *.Cu *.Mask F.SilkS) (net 22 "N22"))
  (pad A10 thru_hole circle (at -16.51 -1.27 270) (size 1.50114 1.50114) (drill 0.8001) (layers *.Cu *.Mask F.SilkS) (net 23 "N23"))
  (pad A9 thru_hole circle (at -19.05 -1.27 270) (size 1.50114 1.50114) (drill 0.8001) (layers *.Cu *.Mask F.SilkS) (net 24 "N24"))
  (pad A8 thru_hole circle (at -21.59 -1.27 270) (size 1.50114 1.50114) (drill 0.8001) (layers *.Cu *.Mask F.SilkS) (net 25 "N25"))
  (pad A7 thru_hole circle (at -24.13 -1.27 270) (size 1.50114 1.50114) (drill 0.8001) (layers *.Cu *.Mask F.SilkS) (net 26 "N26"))
  (pad A6 thru_hole circle (at -26.67 -1.27 270) (size 1.50114 1.50114) (drill 0.8001) (layers *.Cu *.Mask F.SilkS) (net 27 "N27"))
  (pad A5 thru_hole circle (at -29.21 -1.27 270) (size 1.50114 1.50114) (drill 0.8001) (layers *.Cu *.Mask F.SilkS) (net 28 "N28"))
  (pad A4 thru_hole circle (at -31.75 -1.27 270) (size 1.50114 1.50114) (drill 0.8001) (layers *.Cu *.Mask F.SilkS) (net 30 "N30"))
  (pad A3 thru_hole circle (at -34.29 -1.27 270) (size 1.50114 1.50114) (drill 0.8001) (layers *.Cu *.Mask F.SilkS) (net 29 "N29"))
  (pad A2 thru_hole circle (at -36.83 -1.27 270) (size 1.50114 1.50114) (drill 0.8001) (layers *.Cu *.Mask F.SilkS) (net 31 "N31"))
  (pad A1 thru_hole circle (at -39.37 -1.27 270) (size 1.50114 1.50114) (drill 0.8001) (layers *.Cu *.Mask F.SilkS) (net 32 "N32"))
  (pad 1 thru_hole circle (at -44.45 3.81 90) (size 2.90068 2.90068) (drill 2.90068) (layers *.Cu *.Mask F.SilkS))
  (pad 1 thru_hole circle (at 44.45 3.81 90) (size 2.90068 2.90068) (drill 2.90068) (layers *.Cu *.Mask F.SilkS)))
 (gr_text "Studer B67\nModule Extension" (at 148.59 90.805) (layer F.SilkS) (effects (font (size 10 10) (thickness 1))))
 (gr_line (start 50.8 140.64) (end 50.8 40.64) (layer Edge.Cuts) (width 0.15))
 (gr_line (start 250.8 140.64) (end 50.8 140.64) (layer Edge.Cuts) (width 0.15))
 (gr_line (start 250.8 40.64) (end 250.8 140.64) (layer Edge.Cuts) (width 0.15))
 (gr_line (start 50.8 40.64) (end 250.8 40.64) (layer Edge.Cuts) (width 0.15))
 (segment (start 55.88 51.435) (end 245.745 51.435) (width 1) (layer B.Cu) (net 1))
 (segment (start 55.88 53.975) (end 245.745 53.975) (width 1) (layer B.Cu) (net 2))
 (segment (start 55.88 56.515) (end 245.745 56.515) (width 1) (layer B.Cu) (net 3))
 (segment (start 55.88 59.055) (end 245.745 59.055) (width 1) (layer B.Cu) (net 4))
 (segment (start 55.88 61.595) (end 245.745 61.595) (width 1) (layer B.Cu) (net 5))
 (segment (start 55.88 64.135) (end 245.745 64.135) (width 1) (layer B.Cu) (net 6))
 (segment (start 55.88 66.675) (end 245.745 66.675) (width 1) (layer B.Cu) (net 7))
 (segment (start 55.88 69.215) (end 245.745 69.215) (width 1) (layer B.Cu) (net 8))
 (segment (start 55.88 71.755) (end 245.745 71.755) (width 1) (layer B.Cu) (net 9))
 (segment (start 55.88 74.295) (end 245.745 74.295) (width 1) (layer B.Cu) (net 10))
 (segment (start 55.88 76.835) (end 245.745 76.835) (width 1) (layer B.Cu) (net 11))
 (segment (start 55.88 79.375) (end 245.745 79.375) (width 1) (layer B.Cu) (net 12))
 (segment (start 55.88 81.915) (end 245.745 81.915) (width 1) (layer B.Cu) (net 13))
 (segment (start 55.88 84.455) (end 245.745 84.455) (width 1) (layer B.Cu) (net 14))
 (segment (start 55.88 86.995) (end 245.745 86.995) (width 1) (layer B.Cu) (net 15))
 (segment (start 55.88 89.535) (end 245.745 89.535) (width 1) (layer B.Cu) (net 16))
 (segment (start 55.88 92.075) (end 245.745 92.075) (width 1) (layer B.Cu) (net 17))
 (segment (start 55.88 94.615) (end 245.745 94.615) (width 1) (layer B.Cu) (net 18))
 (segment (start 55.88 97.155) (end 245.745 97.155) (width 1) (layer B.Cu) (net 19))
 (segment (start 55.88 99.695) (end 245.745 99.695) (width 1) (layer B.Cu) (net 20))
 (segment (start 55.88 102.235) (end 245.745 102.235) (width 1) (layer B.Cu) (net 21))
 (segment (start 55.88 104.775) (end 245.745 104.775) (width 1) (layer B.Cu) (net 22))
 (segment (start 55.88 107.315) (end 245.745 107.315) (width 1) (layer B.Cu) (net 23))
 (segment (start 55.88 109.855) (end 245.745 109.855) (width 1) (layer B.Cu) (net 24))
 (segment (start 55.88 112.395) (end 245.745 112.395) (width 1) (layer B.Cu) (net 25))
 (segment (start 55.88 114.935) (end 245.745 114.935) (width 1) (layer B.Cu) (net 26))
 (segment (start 55.88 117.475) (end 245.745 117.475) (width 1) (layer B.Cu) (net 27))
 (segment (start 55.88 120.015) (end 245.745 120.015) (width 1) (layer B.Cu) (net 28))
 (segment (start 55.88 125.095) (end 245.745 125.095) (width 1) (layer B.Cu) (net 29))
 (segment (start 55.88 122.555) (end 245.745 122.555) (width 1) (layer B.Cu) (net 30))
 (segment (start 55.88 127.635) (end 245.745 127.635) (width 1) (layer B.Cu) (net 31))
 (segment (start 55.88 130.175) (end 245.745 130.175) (width 1) (layer B.Cu) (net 32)))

